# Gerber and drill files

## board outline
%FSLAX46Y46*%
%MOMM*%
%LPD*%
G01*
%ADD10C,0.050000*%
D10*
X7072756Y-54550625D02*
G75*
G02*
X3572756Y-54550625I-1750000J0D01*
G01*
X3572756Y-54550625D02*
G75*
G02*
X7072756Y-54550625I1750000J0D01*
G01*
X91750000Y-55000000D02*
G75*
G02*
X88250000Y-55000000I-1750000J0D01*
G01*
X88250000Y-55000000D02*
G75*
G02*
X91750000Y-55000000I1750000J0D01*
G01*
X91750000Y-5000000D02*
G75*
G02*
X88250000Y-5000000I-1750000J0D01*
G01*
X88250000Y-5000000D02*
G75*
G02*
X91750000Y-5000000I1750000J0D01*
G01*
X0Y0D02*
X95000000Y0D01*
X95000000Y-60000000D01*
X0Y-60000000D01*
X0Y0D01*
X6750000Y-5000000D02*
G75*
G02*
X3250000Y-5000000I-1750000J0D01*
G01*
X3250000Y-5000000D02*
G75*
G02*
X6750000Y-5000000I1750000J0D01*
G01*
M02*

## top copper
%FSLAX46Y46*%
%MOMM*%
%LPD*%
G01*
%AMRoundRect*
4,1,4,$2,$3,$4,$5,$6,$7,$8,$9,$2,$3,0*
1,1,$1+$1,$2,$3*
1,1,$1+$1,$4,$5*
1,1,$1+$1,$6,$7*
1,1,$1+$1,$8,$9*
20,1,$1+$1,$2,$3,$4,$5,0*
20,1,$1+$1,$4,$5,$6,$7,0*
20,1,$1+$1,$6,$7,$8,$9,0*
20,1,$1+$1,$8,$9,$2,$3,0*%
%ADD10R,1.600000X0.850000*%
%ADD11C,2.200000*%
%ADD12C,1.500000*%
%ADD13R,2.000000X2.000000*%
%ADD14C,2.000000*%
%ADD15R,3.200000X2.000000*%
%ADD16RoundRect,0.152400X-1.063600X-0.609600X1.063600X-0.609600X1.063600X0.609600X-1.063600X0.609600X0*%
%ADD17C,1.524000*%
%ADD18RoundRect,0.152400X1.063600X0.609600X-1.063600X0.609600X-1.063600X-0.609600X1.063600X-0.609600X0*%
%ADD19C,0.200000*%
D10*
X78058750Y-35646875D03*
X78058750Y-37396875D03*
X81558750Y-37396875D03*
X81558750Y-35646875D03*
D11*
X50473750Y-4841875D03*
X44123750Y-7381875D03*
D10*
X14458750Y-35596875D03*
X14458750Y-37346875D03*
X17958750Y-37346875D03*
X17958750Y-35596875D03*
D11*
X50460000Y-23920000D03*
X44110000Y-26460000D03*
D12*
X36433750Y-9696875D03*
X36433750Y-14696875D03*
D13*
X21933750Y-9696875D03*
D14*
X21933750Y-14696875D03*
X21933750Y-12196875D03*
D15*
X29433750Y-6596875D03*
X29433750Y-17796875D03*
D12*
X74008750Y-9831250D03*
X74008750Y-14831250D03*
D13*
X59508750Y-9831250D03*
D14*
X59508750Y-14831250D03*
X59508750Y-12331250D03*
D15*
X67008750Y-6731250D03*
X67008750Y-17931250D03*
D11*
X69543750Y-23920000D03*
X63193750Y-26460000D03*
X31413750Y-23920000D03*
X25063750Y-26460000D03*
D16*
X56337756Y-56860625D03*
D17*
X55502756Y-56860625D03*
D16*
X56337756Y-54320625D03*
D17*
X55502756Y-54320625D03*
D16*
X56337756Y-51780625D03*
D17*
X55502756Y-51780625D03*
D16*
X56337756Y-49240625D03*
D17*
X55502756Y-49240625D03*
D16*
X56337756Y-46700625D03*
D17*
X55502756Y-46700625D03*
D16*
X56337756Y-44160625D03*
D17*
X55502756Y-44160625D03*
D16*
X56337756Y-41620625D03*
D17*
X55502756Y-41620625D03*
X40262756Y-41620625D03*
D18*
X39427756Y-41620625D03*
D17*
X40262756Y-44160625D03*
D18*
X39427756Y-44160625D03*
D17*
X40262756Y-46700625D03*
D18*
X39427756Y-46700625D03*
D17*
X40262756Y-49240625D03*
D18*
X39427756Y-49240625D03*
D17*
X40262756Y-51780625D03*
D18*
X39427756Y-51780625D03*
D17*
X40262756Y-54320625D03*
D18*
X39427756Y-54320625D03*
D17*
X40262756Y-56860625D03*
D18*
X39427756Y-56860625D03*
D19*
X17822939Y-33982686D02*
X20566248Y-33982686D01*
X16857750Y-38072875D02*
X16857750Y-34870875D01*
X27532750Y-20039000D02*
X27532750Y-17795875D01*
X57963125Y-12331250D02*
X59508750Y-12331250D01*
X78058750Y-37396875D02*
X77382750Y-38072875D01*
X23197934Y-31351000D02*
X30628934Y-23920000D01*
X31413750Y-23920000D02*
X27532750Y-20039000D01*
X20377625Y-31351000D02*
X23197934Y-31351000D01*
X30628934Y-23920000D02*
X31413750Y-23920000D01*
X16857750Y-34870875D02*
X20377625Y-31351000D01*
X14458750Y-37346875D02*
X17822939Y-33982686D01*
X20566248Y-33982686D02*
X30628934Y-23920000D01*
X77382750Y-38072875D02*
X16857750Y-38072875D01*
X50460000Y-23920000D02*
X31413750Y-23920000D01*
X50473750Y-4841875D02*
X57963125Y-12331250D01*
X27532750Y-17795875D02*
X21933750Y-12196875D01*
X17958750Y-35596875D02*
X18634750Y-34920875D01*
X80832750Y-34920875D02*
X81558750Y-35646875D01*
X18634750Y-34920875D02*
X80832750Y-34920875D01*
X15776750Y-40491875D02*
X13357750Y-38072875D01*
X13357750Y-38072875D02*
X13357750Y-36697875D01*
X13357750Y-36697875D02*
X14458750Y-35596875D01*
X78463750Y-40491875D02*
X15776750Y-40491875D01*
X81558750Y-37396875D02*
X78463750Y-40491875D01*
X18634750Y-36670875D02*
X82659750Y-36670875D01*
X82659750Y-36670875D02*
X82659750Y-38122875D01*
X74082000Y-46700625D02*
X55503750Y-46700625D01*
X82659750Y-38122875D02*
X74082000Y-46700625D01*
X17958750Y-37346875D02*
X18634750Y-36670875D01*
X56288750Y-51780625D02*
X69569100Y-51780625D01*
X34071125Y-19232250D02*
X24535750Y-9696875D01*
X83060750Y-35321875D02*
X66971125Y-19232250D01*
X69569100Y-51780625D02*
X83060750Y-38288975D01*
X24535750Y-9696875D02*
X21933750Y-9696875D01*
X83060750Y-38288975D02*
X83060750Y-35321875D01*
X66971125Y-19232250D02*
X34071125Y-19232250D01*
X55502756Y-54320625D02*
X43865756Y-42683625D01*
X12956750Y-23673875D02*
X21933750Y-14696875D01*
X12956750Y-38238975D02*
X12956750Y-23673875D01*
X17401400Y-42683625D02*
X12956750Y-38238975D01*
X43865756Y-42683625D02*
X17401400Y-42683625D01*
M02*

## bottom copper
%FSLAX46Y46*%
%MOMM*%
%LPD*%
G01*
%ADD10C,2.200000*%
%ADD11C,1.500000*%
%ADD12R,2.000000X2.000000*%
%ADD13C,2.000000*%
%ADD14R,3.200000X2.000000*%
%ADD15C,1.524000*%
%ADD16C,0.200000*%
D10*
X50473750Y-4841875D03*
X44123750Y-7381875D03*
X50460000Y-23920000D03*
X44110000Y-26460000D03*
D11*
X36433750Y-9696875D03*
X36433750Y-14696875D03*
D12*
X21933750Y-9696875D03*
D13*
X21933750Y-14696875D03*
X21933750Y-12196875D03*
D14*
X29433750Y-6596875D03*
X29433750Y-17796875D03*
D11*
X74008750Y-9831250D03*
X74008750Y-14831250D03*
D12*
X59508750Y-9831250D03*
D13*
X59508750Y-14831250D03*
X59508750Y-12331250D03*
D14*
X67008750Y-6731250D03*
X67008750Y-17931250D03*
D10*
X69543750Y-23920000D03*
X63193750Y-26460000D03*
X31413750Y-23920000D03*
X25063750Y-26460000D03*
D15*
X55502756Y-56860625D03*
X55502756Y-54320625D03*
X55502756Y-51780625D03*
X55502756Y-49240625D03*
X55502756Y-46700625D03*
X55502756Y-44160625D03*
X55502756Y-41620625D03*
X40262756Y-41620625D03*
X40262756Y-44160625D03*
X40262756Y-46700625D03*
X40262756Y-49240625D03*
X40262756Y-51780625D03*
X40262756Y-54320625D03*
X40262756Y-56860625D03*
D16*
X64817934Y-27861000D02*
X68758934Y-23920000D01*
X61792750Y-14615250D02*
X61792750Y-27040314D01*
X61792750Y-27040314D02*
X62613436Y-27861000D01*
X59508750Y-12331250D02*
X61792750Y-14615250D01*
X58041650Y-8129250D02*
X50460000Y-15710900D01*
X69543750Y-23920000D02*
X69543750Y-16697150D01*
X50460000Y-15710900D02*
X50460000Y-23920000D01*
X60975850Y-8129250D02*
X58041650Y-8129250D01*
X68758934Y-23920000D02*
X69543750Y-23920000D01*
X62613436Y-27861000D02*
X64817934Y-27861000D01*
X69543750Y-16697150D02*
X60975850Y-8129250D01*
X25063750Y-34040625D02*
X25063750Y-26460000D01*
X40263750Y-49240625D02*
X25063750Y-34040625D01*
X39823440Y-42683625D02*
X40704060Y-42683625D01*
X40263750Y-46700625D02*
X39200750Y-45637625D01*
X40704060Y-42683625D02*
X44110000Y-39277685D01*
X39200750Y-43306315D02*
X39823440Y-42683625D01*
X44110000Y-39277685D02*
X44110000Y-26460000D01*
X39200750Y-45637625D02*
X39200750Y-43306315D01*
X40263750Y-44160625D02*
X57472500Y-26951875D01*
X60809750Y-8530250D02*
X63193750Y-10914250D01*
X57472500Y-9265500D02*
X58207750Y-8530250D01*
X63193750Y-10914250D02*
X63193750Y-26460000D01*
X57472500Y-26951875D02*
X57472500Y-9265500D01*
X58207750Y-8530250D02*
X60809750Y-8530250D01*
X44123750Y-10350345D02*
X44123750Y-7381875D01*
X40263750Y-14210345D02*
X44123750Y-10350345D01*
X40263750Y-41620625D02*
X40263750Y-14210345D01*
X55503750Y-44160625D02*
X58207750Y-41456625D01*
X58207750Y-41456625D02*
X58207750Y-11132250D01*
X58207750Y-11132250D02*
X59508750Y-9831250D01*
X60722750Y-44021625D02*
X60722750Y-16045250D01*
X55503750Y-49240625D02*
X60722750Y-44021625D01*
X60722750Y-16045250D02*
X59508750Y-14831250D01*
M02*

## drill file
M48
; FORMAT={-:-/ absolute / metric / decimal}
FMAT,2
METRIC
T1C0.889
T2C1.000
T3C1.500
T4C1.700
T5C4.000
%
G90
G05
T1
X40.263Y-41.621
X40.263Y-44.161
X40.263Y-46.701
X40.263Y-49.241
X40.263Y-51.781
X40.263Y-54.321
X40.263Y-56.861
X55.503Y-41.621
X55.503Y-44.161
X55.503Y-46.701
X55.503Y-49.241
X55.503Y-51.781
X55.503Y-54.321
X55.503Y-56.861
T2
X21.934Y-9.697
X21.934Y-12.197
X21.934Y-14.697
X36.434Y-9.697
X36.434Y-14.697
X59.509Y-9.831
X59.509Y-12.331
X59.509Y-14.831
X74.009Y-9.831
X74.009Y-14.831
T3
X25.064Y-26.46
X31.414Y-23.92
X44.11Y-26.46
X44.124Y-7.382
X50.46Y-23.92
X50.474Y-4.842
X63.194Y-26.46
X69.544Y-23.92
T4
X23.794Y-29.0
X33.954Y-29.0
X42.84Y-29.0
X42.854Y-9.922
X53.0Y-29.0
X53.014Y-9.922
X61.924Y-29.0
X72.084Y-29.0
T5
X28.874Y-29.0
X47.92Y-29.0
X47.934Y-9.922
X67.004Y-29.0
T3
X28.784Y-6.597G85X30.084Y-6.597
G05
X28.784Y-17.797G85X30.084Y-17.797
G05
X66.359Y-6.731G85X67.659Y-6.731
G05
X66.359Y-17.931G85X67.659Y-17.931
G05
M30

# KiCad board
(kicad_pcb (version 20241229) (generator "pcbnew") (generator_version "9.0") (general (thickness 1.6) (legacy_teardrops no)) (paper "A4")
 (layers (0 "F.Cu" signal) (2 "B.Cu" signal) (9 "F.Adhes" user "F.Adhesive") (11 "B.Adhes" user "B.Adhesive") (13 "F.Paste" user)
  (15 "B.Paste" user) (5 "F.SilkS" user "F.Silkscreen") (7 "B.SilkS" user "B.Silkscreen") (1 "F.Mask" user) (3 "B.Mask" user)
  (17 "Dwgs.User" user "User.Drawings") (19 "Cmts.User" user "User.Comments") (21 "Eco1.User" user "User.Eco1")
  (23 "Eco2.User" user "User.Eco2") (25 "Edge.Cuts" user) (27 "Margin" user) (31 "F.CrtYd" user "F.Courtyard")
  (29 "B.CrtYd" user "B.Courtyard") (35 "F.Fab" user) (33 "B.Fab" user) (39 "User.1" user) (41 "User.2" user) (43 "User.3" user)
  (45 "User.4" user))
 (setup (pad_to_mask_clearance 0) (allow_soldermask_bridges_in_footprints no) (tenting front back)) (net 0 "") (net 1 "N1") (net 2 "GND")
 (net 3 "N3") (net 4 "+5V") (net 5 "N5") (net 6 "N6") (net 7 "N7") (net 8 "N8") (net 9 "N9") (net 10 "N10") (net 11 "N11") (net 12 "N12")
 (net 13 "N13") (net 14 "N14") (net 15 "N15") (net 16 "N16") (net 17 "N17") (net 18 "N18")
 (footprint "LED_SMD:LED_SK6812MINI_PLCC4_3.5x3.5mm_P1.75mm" (layer "F.Cu") (at 79.80875 36.521875)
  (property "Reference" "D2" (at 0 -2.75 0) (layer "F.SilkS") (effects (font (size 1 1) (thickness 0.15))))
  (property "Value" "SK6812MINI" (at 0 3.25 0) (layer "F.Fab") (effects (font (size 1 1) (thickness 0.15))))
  (pad "1" smd rect (at -1.75 -0.875) (size 1.6 0.85) (layers "F.Cu" "F.Mask" "F.Paste") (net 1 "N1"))
  (pad "2" smd rect (at -1.75 0.875) (size 1.6 0.85) (layers "F.Cu" "F.Mask" "F.Paste") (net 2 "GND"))
  (pad "3" smd rect (at 1.75 0.875) (size 1.6 0.85) (layers "F.Cu" "F.Mask" "F.Paste") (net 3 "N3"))
  (pad "4" smd rect (at 1.75 -0.875) (size 1.6 0.85) (layers "F.Cu" "F.Mask" "F.Paste") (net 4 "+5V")))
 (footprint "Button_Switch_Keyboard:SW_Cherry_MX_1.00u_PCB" (layer "F.Cu") (at 50.47375 4.841875)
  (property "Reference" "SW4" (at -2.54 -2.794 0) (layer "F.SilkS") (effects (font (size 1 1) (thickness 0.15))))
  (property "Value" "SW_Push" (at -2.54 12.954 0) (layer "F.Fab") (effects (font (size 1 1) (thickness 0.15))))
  (pad "" np_thru_hole circle (at -7.62 5.08) (size 1.7 1.7) (drill 1.7) (layers "*.Cu" "*.Mask"))
  (pad "" np_thru_hole circle (at -2.54 5.08) (size 4 4) (drill 4) (layers "*.Cu" "*.Mask"))
  (pad "" np_thru_hole circle (at 2.54 5.08) (size 1.7 1.7) (drill 1.7) (layers "*.Cu" "*.Mask"))
  (pad "1" thru_hole circle (at 0 0) (size 2.2 2.2) (drill 1.5) (layers "*.Cu" "*.Mask") (remove_unused_layers no) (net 2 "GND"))
  (pad "2" thru_hole circle (at -6.35 2.54) (size 2.2 2.2) (drill 1.5) (layers "*.Cu" "*.Mask") (remove_unused_layers no) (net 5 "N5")))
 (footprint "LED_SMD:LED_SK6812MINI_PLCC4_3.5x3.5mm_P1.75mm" (layer "F.Cu") (at 16.20875 36.471875)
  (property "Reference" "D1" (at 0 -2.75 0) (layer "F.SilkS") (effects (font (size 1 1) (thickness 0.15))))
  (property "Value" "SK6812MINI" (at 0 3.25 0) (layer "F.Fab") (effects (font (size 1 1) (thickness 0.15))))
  (pad "1" smd rect (at -1.75 -0.875) (size 1.6 0.85) (layers "F.Cu" "F.Mask" "F.Paste") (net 3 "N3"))
  (pad "2" smd rect (at -1.75 0.875) (size 1.6 0.85) (layers "F.Cu" "F.Mask" "F.Paste") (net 2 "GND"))
  (pad "3" smd rect (at 1.75 0.875) (size 1.6 0.85) (layers "F.Cu" "F.Mask" "F.Paste") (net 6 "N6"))
  (pad "4" smd rect (at 1.75 -0.875) (size 1.6 0.85) (layers "F.Cu" "F.Mask" "F.Paste") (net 4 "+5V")))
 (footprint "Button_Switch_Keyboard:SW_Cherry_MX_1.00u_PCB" (layer "F.Cu") (at 50.46 23.92)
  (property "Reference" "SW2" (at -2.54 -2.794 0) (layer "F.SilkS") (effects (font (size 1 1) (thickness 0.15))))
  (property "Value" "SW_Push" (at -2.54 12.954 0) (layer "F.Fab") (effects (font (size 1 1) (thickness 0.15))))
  (pad "" np_thru_hole circle (at -7.62 5.08) (size 1.7 1.7) (drill 1.7) (layers "*.Cu" "*.Mask"))
  (pad "" np_thru_hole circle (at -2.54 5.08) (size 4 4) (drill 4) (layers "*.Cu" "*.Mask"))
  (pad "" np_thru_hole circle (at 2.54 5.08) (size 1.7 1.7) (drill 1.7) (layers "*.Cu" "*.Mask"))
  (pad "1" thru_hole circle (at 0 0) (size 2.2 2.2) (drill 1.5) (layers "*.Cu" "*.Mask") (remove_unused_layers no) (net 2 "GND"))
  (pad "2" thru_hole circle (at -6.35 2.54) (size 2.2 2.2) (drill 1.5) (layers "*.Cu" "*.Mask") (remove_unused_layers no) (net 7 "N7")))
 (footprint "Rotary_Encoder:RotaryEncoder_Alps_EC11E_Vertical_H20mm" (layer "F.Cu") (at 21.93375 9.696875)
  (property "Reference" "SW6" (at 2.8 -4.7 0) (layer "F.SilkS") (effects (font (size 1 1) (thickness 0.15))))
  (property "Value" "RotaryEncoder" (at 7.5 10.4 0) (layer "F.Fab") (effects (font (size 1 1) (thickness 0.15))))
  (pad "" thru_hole circle (at 14.5 0) (size 1.5 1.5) (drill 1) (layers "*.Cu" "*.Mask") (remove_unused_layers no))
  (pad "" thru_hole circle (at 14.5 5) (size 1.5 1.5) (drill 1) (layers "*.Cu" "*.Mask") (remove_unused_layers no))
  (pad "A" thru_hole rect (at 0 0) (size 2 2) (drill 1) (layers "*.Cu" "*.Mask") (remove_unused_layers no) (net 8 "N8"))
  (pad "B" thru_hole circle (at 0 5) (size 2 2) (drill 1) (layers "*.Cu" "*.Mask") (remove_unused_layers no) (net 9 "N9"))
  (pad "C" thru_hole circle (at 0 2.5) (size 2 2) (drill 1) (layers "*.Cu" "*.Mask") (remove_unused_layers no) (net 2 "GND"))
  (pad "MP" thru_hole rect (at 7.5 -3.1) (size 3.2 2) (drill oval 2.8 1.5) (layers "*.Cu" "*.Mask") (remove_unused_layers no))
  (pad "MP" thru_hole rect (at 7.5 8.1) (size 3.2 2) (drill oval 2.8 1.5) (layers "*.Cu" "*.Mask") (remove_unused_layers no)))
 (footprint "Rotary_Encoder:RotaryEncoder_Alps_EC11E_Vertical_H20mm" (layer "F.Cu") (at 59.50875 9.83125)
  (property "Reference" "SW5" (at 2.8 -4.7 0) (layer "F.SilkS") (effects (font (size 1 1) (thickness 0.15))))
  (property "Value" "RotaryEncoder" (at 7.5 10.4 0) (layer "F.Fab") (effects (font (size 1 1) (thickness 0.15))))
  (pad "" thru_hole circle (at 14.5 0) (size 1.5 1.5) (drill 1) (layers "*.Cu" "*.Mask") (remove_unused_layers no))
  (pad "" thru_hole circle (at 14.5 5) (size 1.5 1.5) (drill 1) (layers "*.Cu" "*.Mask") (remove_unused_layers no))
  (pad "A" thru_hole rect (at 0 0) (size 2 2) (drill 1) (layers "*.Cu" "*.Mask") (remove_unused_layers no) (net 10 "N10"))
  (pad "B" thru_hole circle (at 0 5) (size 2 2) (drill 1) (layers "*.Cu" "*.Mask") (remove_unused_layers no) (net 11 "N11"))
  (pad "C" thru_hole circle (at 0 2.5) (size 2 2) (drill 1) (layers "*.Cu" "*.Mask") (remove_unused_layers no) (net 2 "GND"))
  (pad "MP" thru_hole rect (at 7.5 -3.1) (size 3.2 2) (drill oval 2.8 1.5) (layers "*.Cu" "*.Mask") (remove_unused_layers no))
  (pad "MP" thru_hole rect (at 7.5 8.1) (size 3.2 2) (drill oval 2.8 1.5) (layers "*.Cu" "*.Mask") (remove_unused_layers no)))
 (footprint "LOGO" (layer "F.Cu") (at 47.5 32.800625)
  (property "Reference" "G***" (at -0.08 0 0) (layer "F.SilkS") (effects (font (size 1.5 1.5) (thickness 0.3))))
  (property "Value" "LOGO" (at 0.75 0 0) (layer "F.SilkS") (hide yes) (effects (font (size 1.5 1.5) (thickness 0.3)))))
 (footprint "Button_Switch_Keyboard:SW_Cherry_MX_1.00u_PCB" (layer "F.Cu") (at 69.54375 23.92)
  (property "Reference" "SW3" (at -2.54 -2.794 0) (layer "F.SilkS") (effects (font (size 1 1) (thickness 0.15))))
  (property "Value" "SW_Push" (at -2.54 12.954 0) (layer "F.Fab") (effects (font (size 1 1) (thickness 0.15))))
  (pad "" np_thru_hole circle (at -7.62 5.08) (size 1.7 1.7) (drill 1.7) (layers "*.Cu" "*.Mask"))
  (pad "" np_thru_hole circle (at -2.54 5.08) (size 4 4) (drill 4) (layers "*.Cu" "*.Mask"))
  (pad "" np_thru_hole circle (at 2.54 5.08) (size 1.7 1.7) (drill 1.7) (layers "*.Cu" "*.Mask"))
  (pad "1" thru_hole circle (at 0 0) (size 2.2 2.2) (drill 1.5) (layers "*.Cu" "*.Mask") (remove_unused_layers no) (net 2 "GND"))
  (pad "2" thru_hole circle (at -6.35 2.54) (size 2.2 2.2) (drill 1.5) (layers "*.Cu" "*.Mask") (remove_unused_layers no) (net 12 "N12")))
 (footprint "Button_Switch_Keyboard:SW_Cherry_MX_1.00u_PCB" (layer "F.Cu") (at 31.41375 23.92)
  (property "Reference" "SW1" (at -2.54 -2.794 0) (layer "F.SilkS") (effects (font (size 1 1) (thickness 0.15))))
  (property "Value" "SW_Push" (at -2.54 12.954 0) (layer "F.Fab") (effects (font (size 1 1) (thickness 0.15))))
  (pad "" np_thru_hole circle (at -7.62 5.08) (size 1.7 1.7) (drill 1.7) (layers "*.Cu" "*.Mask"))
  (pad "" np_thru_hole circle (at -2.54 5.08) (size 4 4) (drill 4) (layers "*.Cu" "*.Mask"))
  (pad "" np_thru_hole circle (at 2.54 5.08) (size 1.7 1.7) (drill 1.7) (layers "*.Cu" "*.Mask"))
  (pad "1" thru_hole circle (at 0 0) (size 2.2 2.2) (drill 1.5) (layers "*.Cu" "*.Mask") (remove_unused_layers no) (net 2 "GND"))
  (pad "2" thru_hole circle (at -6.35 2.54) (size 2.2 2.2) (drill 1.5) (layers "*.Cu" "*.Mask") (remove_unused_layers no) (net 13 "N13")))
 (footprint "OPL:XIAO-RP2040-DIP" (layer "F.Cu") (at 47.882756 49.240625 180)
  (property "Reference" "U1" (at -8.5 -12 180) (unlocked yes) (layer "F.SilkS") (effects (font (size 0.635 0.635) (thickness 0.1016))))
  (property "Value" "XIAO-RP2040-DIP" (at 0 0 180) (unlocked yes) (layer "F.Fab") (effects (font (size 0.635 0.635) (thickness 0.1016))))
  (pad "1" smd roundrect (at -8.455 -7.62) (size 2.432 1.524) (layers "F.Cu" "F.Mask") (roundrect_rratio 0.1) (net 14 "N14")
   (thermal_bridge_angle 45))
  (pad "1" thru_hole circle (at -7.62 -7.62) (size 1.524 1.524) (drill 0.889) (layers "*.Cu" "*.Mask") (remove_unused_layers no)
   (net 14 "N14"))
  (pad "2" smd roundrect (at -8.455 -5.08) (size 2.432 1.524) (layers "F.Cu" "F.Mask") (roundrect_rratio 0.1) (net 9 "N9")
   (thermal_bridge_angle 45))
  (pad "2" thru_hole circle (at -7.62 -5.08) (size 1.524 1.524) (drill 0.889) (layers "*.Cu" "*.Mask") (remove_unused_layers no)
   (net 9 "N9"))
  (pad "3" smd roundrect (at -8.455 -2.54) (size 2.432 1.524) (layers "F.Cu" "F.Mask") (roundrect_rratio 0.1) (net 8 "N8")
   (thermal_bridge_angle 45))
  (pad "3" thru_hole circle (at -7.62 -2.54) (size 1.524 1.524) (drill 0.889) (layers "*.Cu" "*.Mask") (remove_unused_layers no)
   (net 8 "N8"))
  (pad "4" smd roundrect (at -8.455 0) (size 2.432 1.524) (layers "F.Cu" "F.Mask") (roundrect_rratio 0.1) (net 11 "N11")
   (thermal_bridge_angle 45))
  (pad "4" thru_hole circle (at -7.62 0) (size 1.524 1.524) (drill 0.889) (layers "*.Cu" "*.Mask") (remove_unused_layers no) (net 11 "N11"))
  (pad "5" smd roundrect (at -8.455 2.54) (size 2.432 1.524) (layers "F.Cu" "F.Mask") (roundrect_rratio 0.1) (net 6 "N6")
   (thermal_bridge_angle 45))
  (pad "5" thru_hole circle (at -7.62 2.54) (size 1.524 1.524) (drill 0.889) (layers "*.Cu" "*.Mask") (remove_unused_layers no) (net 6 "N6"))
  (pad "6" smd roundrect (at -8.455 5.08) (size 2.432 1.524) (layers "F.Cu" "F.Mask") (roundrect_rratio 0.1) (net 10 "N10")
   (thermal_bridge_angle 45))
  (pad "6" thru_hole circle (at -7.62 5.08) (size 1.524 1.524) (drill 0.889) (layers "*.Cu" "*.Mask") (remove_unused_layers no)
   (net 10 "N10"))
  (pad "7" smd roundrect (at -8.455 7.62) (size 2.432 1.524) (layers "F.Cu" "F.Mask") (roundrect_rratio 0.1) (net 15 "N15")
   (thermal_bridge_angle 45))
  (pad "7" thru_hole circle (at -7.62 7.62) (size 1.524 1.524) (drill 0.889) (layers "*.Cu" "*.Mask") (remove_unused_layers no)
   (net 15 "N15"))
  (pad "8" thru_hole circle (at 7.62 7.62 180) (size 1.524 1.524) (drill 0.889) (layers "*.Cu" "*.Mask") (remove_unused_layers no)
   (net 5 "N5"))
  (pad "8" smd roundrect (at 8.455 7.62 180) (size 2.432 1.524) (layers "F.Cu" "F.Mask") (roundrect_rratio 0.1) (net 5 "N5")
   (thermal_bridge_angle 45))
  (pad "9" thru_hole circle (at 7.62 5.08 180) (size 1.524 1.524) (drill 0.889) (layers "*.Cu" "*.Mask") (remove_unused_layers no)
   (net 12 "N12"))
  (pad "9" smd roundrect (at 8.455 5.08 180) (size 2.432 1.524) (layers "F.Cu" "F.Mask") (roundrect_rratio 0.1) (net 12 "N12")
   (thermal_bridge_angle 45))
  (pad "10" thru_hole circle (at 7.62 2.54 180) (size 1.524 1.524) (drill 0.889) (layers "*.Cu" "*.Mask") (remove_unused_layers no)
   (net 7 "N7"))
  (pad "10" smd roundrect (at 8.455 2.54 180) (size 2.432 1.524) (layers "F.Cu" "F.Mask") (roundrect_rratio 0.1) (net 7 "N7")
   (thermal_bridge_angle 45))
  (pad "11" thru_hole circle (at 7.62 0 180) (size 1.524 1.524) (drill 0.889) (layers "*.Cu" "*.Mask") (remove_unused_layers no)
   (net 13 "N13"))
  (pad "11" smd roundrect (at 8.455 0 180) (size 2.432 1.524) (layers "F.Cu" "F.Mask") (roundrect_rratio 0.1) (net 13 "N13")
   (thermal_bridge_angle 45))
  (pad "12" thru_hole circle (at 7.62 -2.54 180) (size 1.524 1.524) (drill 0.889) (layers "*.Cu" "*.Mask") (remove_unused_layers no)
   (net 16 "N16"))
  (pad "12" smd roundrect (at 8.455 -2.54 180) (size 2.432 1.524) (layers "F.Cu" "F.Mask") (roundrect_rratio 0.1) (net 16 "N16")
   (thermal_bridge_angle 45))
  (pad "13" thru_hole circle (at 7.62 -5.08 180) (size 1.524 1.524) (drill 0.889) (layers "*.Cu" "*.Mask") (remove_unused_layers no)
   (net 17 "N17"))
  (pad "13" smd roundrect (at 8.455 -5.08 180) (size 2.432 1.524) (layers "F.Cu" "F.Mask") (roundrect_rratio 0.1) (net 17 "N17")
   (thermal_bridge_angle 45))
  (pad "14" thru_hole circle (at 7.62 -7.62 180) (size 1.524 1.524) (drill 0.889) (layers "*.Cu" "*.Mask") (remove_unused_layers no)
   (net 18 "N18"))
  (pad "14" smd roundrect (at 8.455 -7.62 180) (size 2.432 1.524) (layers "F.Cu" "F.Mask") (roundrect_rratio 0.1) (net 18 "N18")
   (thermal_bridge_angle 45)))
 (gr_circle (center 5.322756 54.550625) (end 7.072756 54.550625) (stroke (width 0.05) (type solid)) (fill no) (layer "Edge.Cuts"))
 (gr_circle (center 90 55) (end 91.75 55) (stroke (width 0.05) (type solid)) (fill no) (layer "Edge.Cuts"))
 (gr_circle (center 90 5) (end 91.75 5) (stroke (width 0.05) (type solid)) (fill no) (layer "Edge.Cuts"))
 (gr_rect (start 0 0) (end 95 60) (stroke (width 0.05) (type solid)) (fill no) (layer "Edge.Cuts"))
 (gr_circle (center 5 5) (end 6.75 5) (stroke (width 0.05) (type solid)) (fill no) (layer "Edge.Cuts"))
 (segment (start 17.822939 33.982686) (end 20.566248 33.982686) (width 0.2) (layer "F.Cu") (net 2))
 (segment (start 16.85775 38.072875) (end 16.85775 34.870875) (width 0.2) (layer "F.Cu") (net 2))
 (segment (start 27.53275 20.039) (end 27.53275 17.795875) (width 0.2) (layer "F.Cu") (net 2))
 (segment (start 57.963125 12.33125) (end 59.50875 12.33125) (width 0.2) (layer "F.Cu") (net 2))
 (segment (start 78.05875 37.396875) (end 77.38275 38.072875) (width 0.2) (layer "F.Cu") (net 2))
 (segment (start 23.197934 31.351) (end 30.628934 23.92) (width 0.2) (layer "F.Cu") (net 2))
 (segment (start 31.41375 23.92) (end 27.53275 20.039) (width 0.2) (layer "F.Cu") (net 2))
 (segment (start 20.377625 31.351) (end 23.197934 31.351) (width 0.2) (layer "F.Cu") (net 2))
 (segment (start 30.628934 23.92) (end 31.41375 23.92) (width 0.2) (layer "F.Cu") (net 2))
 (segment (start 16.85775 34.870875) (end 20.377625 31.351) (width 0.2) (layer "F.Cu") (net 2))
 (segment (start 14.45875 37.346875) (end 17.822939 33.982686) (width 0.2) (layer "F.Cu") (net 2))
 (segment (start 20.566248 33.982686) (end 30.628934 23.92) (width 0.2) (layer "F.Cu") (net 2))
 (segment (start 77.38275 38.072875) (end 16.85775 38.072875) (width 0.2) (layer "F.Cu") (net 2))
 (segment (start 50.46 23.92) (end 31.41375 23.92) (width 0.2) (layer "F.Cu") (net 2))
 (segment (start 50.47375 4.841875) (end 57.963125 12.33125) (width 0.2) (layer "F.Cu") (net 2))
 (segment (start 27.53275 17.795875) (end 21.93375 12.196875) (width 0.2) (layer "F.Cu") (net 2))
 (segment (start 64.817934 27.861) (end 68.758934 23.92) (width 0.2) (layer "B.Cu") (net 2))
 (segment (start 61.79275 14.61525) (end 61.79275 27.040314) (width 0.2) (layer "B.Cu") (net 2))
 (segment (start 61.79275 27.040314) (end 62.613436 27.861) (width 0.2) (layer "B.Cu") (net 2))
 (segment (start 59.50875 12.33125) (end 61.79275 14.61525) (width 0.2) (layer "B.Cu") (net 2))
 (segment (start 58.04165 8.12925) (end 50.46 15.7109) (width 0.2) (layer "B.Cu") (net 2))
 (segment (start 69.54375 23.92) (end 69.54375 16.69715) (width 0.2) (layer "B.Cu") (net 2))
 (segment (start 50.46 15.7109) (end 50.46 23.92) (width 0.2) (layer "B.Cu") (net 2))
 (segment (start 60.97585 8.12925) (end 58.04165 8.12925) (width 0.2) (layer "B.Cu") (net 2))
 (segment (start 68.758934 23.92) (end 69.54375 23.92) (width 0.2) (layer "B.Cu") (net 2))
 (segment (start 62.613436 27.861) (end 64.817934 27.861) (width 0.2) (layer "B.Cu") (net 2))
 (segment (start 69.54375 16.69715) (end 60.97585 8.12925) (width 0.2) (layer "B.Cu") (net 2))
 (segment (start 17.95875 35.596875) (end 18.63475 34.920875) (width 0.2) (layer "F.Cu") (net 4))
 (segment (start 80.83275 34.920875) (end 81.55875 35.646875) (width 0.2) (layer "F.Cu") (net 4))
 (segment (start 18.63475 34.920875) (end 80.83275 34.920875) (width 0.2) (layer "F.Cu") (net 4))
 (segment (start 15.77675 40.491875) (end 13.35775 38.072875) (width 0.2) (layer "F.Cu") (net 3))
 (segment (start 13.35775 38.072875) (end 13.35775 36.697875) (width 0.2) (layer "F.Cu") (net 3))
 (segment (start 13.35775 36.697875) (end 14.45875 35.596875) (width 0.2) (layer "F.Cu") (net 3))
 (segment (start 78.46375 40.491875) (end 15.77675 40.491875) (width 0.2) (layer "F.Cu") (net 3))
 (segment (start 81.55875 37.396875) (end 78.46375 40.491875) (width 0.2) (layer "F.Cu") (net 3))
 (segment (start 18.63475 36.670875) (end 82.65975 36.670875) (width 0.2) (layer "F.Cu") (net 6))
 (segment (start 82.65975 36.670875) (end 82.65975 38.122875) (width 0.2) (layer "F.Cu") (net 6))
 (segment (start 74.082 46.700625) (end 55.50375 46.700625) (width 0.2) (layer "F.Cu") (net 6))
 (segment (start 82.65975 38.122875) (end 74.082 46.700625) (width 0.2) (layer "F.Cu") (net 6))
 (segment (start 17.95875 37.346875) (end 18.63475 36.670875) (width 0.2) (layer "F.Cu") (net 6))
 (segment (start 25.06375 34.040625) (end 25.06375 26.46) (width 0.2) (layer "B.Cu") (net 13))
 (segment (start 40.26375 49.240625) (end 25.06375 34.040625) (width 0.2) (layer "B.Cu") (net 13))
 (segment (start 39.82344 42.683625) (end 40.70406 42.683625) (width 0.2) (layer "B.Cu") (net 7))
 (segment (start 40.26375 46.700625) (end 39.20075 45.637625) (width 0.2) (layer "B.Cu") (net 7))
 (segment (start 40.70406 42.683625) (end 44.11 39.277685) (width 0.2) (layer "B.Cu") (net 7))
 (segment (start 39.20075 43.306315) (end 39.82344 42.683625) (width 0.2) (layer "B.Cu") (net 7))
 (segment (start 44.11 39.277685) (end 44.11 26.46) (width 0.2) (layer "B.Cu") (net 7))
 (segment (start 39.20075 45.637625) (end 39.20075 43.306315) (width 0.2) (layer "B.Cu") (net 7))
 (segment (start 40.26375 44.160625) (end 57.4725 26.951875) (width 0.2) (layer "B.Cu") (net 12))
 (segment (start 60.80975 8.53025) (end 63.19375 10.91425) (width 0.2) (layer "B.Cu") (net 12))
 (segment (start 57.4725 9.2655) (end 58.20775 8.53025) (width 0.2) (layer "B.Cu") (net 12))
 (segment (start 63.19375 10.91425) (end 63.19375 26.46) (width 0.2) (layer "B.Cu") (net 12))
 (segment (start 57.4725 26.951875) (end 57.4725 9.2655) (width 0.2) (layer "B.Cu") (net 12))
 (segment (start 58.20775 8.53025) (end 60.80975 8.53025) (width 0.2) (layer "B.Cu") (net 12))
 (segment (start 44.12375 10.350345) (end 44.12375 7.381875) (width 0.2) (layer "B.Cu") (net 5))
 (segment (start 40.26375 14.210345) (end 44.12375 10.350345) (width 0.2) (layer "B.Cu") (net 5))
 (segment (start 40.26375 41.620625) (end 40.26375 14.210345) (width 0.2) (layer "B.Cu") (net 5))
 (segment (start 56.28875 51.780625) (end 69.5691 51.780625) (width 0.2) (layer "F.Cu") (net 8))
 (segment (start 34.071125 19.23225) (end 24.53575 9.696875) (width 0.2) (layer "F.Cu") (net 8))
 (segment (start 83.06075 35.321875) (end 66.971125 19.23225) (width 0.2) (layer "F.Cu") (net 8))
 (segment (start 69.5691 51.780625) (end 83.06075 38.288975) (width 0.2) (layer "F.Cu") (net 8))
 (segment (start 24.53575 9.696875) (end 21.93375 9.696875) (width 0.2) (layer "F.Cu") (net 8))
 (segment (start 83.06075 38.288975) (end 83.06075 35.321875) (width 0.2) (layer "F.Cu") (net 8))
 (segment (start 66.971125 19.23225) (end 34.071125 19.23225) (width 0.2) (layer "F.Cu") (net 8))
 (segment (start 55.50375 44.160625) (end 58.20775 41.456625) (width 0.2) (layer "B.Cu") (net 10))
 (segment (start 58.20775 41.456625) (end 58.20775 11.13225) (width 0.2) (layer "B.Cu") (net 10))
 (segment (start 58.20775 11.13225) (end 59.50875 9.83125) (width 0.2) (layer "B.Cu") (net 10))
 (segment (start 60.72275 44.021625) (end 60.72275 16.04525) (width 0.2) (layer "B.Cu") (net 11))
 (segment (start 55.50375 49.240625) (end 60.72275 44.021625) (width 0.2) (layer "B.Cu") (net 11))
 (segment (start 60.72275 16.04525) (end 59.50875 14.83125) (width 0.2) (layer "B.Cu") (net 11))
 (segment (start 55.502756 54.320625) (end 43.865756 42.683625) (width 0.2) (layer "F.Cu") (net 9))
 (segment (start 12.95675 23.673875) (end 21.93375 14.696875) (width 0.2) (layer "F.Cu") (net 9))
 (segment (start 12.95675 38.238975) (end 12.95675 23.673875) (width 0.2) (layer "F.Cu") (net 9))
 (segment (start 17.4014 42.683625) (end 12.95675 38.238975) (width 0.2) (layer "F.Cu") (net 9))
 (segment (start 43.865756 42.683625) (end 17.4014 42.683625) (width 0.2) (layer "F.Cu") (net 9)))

